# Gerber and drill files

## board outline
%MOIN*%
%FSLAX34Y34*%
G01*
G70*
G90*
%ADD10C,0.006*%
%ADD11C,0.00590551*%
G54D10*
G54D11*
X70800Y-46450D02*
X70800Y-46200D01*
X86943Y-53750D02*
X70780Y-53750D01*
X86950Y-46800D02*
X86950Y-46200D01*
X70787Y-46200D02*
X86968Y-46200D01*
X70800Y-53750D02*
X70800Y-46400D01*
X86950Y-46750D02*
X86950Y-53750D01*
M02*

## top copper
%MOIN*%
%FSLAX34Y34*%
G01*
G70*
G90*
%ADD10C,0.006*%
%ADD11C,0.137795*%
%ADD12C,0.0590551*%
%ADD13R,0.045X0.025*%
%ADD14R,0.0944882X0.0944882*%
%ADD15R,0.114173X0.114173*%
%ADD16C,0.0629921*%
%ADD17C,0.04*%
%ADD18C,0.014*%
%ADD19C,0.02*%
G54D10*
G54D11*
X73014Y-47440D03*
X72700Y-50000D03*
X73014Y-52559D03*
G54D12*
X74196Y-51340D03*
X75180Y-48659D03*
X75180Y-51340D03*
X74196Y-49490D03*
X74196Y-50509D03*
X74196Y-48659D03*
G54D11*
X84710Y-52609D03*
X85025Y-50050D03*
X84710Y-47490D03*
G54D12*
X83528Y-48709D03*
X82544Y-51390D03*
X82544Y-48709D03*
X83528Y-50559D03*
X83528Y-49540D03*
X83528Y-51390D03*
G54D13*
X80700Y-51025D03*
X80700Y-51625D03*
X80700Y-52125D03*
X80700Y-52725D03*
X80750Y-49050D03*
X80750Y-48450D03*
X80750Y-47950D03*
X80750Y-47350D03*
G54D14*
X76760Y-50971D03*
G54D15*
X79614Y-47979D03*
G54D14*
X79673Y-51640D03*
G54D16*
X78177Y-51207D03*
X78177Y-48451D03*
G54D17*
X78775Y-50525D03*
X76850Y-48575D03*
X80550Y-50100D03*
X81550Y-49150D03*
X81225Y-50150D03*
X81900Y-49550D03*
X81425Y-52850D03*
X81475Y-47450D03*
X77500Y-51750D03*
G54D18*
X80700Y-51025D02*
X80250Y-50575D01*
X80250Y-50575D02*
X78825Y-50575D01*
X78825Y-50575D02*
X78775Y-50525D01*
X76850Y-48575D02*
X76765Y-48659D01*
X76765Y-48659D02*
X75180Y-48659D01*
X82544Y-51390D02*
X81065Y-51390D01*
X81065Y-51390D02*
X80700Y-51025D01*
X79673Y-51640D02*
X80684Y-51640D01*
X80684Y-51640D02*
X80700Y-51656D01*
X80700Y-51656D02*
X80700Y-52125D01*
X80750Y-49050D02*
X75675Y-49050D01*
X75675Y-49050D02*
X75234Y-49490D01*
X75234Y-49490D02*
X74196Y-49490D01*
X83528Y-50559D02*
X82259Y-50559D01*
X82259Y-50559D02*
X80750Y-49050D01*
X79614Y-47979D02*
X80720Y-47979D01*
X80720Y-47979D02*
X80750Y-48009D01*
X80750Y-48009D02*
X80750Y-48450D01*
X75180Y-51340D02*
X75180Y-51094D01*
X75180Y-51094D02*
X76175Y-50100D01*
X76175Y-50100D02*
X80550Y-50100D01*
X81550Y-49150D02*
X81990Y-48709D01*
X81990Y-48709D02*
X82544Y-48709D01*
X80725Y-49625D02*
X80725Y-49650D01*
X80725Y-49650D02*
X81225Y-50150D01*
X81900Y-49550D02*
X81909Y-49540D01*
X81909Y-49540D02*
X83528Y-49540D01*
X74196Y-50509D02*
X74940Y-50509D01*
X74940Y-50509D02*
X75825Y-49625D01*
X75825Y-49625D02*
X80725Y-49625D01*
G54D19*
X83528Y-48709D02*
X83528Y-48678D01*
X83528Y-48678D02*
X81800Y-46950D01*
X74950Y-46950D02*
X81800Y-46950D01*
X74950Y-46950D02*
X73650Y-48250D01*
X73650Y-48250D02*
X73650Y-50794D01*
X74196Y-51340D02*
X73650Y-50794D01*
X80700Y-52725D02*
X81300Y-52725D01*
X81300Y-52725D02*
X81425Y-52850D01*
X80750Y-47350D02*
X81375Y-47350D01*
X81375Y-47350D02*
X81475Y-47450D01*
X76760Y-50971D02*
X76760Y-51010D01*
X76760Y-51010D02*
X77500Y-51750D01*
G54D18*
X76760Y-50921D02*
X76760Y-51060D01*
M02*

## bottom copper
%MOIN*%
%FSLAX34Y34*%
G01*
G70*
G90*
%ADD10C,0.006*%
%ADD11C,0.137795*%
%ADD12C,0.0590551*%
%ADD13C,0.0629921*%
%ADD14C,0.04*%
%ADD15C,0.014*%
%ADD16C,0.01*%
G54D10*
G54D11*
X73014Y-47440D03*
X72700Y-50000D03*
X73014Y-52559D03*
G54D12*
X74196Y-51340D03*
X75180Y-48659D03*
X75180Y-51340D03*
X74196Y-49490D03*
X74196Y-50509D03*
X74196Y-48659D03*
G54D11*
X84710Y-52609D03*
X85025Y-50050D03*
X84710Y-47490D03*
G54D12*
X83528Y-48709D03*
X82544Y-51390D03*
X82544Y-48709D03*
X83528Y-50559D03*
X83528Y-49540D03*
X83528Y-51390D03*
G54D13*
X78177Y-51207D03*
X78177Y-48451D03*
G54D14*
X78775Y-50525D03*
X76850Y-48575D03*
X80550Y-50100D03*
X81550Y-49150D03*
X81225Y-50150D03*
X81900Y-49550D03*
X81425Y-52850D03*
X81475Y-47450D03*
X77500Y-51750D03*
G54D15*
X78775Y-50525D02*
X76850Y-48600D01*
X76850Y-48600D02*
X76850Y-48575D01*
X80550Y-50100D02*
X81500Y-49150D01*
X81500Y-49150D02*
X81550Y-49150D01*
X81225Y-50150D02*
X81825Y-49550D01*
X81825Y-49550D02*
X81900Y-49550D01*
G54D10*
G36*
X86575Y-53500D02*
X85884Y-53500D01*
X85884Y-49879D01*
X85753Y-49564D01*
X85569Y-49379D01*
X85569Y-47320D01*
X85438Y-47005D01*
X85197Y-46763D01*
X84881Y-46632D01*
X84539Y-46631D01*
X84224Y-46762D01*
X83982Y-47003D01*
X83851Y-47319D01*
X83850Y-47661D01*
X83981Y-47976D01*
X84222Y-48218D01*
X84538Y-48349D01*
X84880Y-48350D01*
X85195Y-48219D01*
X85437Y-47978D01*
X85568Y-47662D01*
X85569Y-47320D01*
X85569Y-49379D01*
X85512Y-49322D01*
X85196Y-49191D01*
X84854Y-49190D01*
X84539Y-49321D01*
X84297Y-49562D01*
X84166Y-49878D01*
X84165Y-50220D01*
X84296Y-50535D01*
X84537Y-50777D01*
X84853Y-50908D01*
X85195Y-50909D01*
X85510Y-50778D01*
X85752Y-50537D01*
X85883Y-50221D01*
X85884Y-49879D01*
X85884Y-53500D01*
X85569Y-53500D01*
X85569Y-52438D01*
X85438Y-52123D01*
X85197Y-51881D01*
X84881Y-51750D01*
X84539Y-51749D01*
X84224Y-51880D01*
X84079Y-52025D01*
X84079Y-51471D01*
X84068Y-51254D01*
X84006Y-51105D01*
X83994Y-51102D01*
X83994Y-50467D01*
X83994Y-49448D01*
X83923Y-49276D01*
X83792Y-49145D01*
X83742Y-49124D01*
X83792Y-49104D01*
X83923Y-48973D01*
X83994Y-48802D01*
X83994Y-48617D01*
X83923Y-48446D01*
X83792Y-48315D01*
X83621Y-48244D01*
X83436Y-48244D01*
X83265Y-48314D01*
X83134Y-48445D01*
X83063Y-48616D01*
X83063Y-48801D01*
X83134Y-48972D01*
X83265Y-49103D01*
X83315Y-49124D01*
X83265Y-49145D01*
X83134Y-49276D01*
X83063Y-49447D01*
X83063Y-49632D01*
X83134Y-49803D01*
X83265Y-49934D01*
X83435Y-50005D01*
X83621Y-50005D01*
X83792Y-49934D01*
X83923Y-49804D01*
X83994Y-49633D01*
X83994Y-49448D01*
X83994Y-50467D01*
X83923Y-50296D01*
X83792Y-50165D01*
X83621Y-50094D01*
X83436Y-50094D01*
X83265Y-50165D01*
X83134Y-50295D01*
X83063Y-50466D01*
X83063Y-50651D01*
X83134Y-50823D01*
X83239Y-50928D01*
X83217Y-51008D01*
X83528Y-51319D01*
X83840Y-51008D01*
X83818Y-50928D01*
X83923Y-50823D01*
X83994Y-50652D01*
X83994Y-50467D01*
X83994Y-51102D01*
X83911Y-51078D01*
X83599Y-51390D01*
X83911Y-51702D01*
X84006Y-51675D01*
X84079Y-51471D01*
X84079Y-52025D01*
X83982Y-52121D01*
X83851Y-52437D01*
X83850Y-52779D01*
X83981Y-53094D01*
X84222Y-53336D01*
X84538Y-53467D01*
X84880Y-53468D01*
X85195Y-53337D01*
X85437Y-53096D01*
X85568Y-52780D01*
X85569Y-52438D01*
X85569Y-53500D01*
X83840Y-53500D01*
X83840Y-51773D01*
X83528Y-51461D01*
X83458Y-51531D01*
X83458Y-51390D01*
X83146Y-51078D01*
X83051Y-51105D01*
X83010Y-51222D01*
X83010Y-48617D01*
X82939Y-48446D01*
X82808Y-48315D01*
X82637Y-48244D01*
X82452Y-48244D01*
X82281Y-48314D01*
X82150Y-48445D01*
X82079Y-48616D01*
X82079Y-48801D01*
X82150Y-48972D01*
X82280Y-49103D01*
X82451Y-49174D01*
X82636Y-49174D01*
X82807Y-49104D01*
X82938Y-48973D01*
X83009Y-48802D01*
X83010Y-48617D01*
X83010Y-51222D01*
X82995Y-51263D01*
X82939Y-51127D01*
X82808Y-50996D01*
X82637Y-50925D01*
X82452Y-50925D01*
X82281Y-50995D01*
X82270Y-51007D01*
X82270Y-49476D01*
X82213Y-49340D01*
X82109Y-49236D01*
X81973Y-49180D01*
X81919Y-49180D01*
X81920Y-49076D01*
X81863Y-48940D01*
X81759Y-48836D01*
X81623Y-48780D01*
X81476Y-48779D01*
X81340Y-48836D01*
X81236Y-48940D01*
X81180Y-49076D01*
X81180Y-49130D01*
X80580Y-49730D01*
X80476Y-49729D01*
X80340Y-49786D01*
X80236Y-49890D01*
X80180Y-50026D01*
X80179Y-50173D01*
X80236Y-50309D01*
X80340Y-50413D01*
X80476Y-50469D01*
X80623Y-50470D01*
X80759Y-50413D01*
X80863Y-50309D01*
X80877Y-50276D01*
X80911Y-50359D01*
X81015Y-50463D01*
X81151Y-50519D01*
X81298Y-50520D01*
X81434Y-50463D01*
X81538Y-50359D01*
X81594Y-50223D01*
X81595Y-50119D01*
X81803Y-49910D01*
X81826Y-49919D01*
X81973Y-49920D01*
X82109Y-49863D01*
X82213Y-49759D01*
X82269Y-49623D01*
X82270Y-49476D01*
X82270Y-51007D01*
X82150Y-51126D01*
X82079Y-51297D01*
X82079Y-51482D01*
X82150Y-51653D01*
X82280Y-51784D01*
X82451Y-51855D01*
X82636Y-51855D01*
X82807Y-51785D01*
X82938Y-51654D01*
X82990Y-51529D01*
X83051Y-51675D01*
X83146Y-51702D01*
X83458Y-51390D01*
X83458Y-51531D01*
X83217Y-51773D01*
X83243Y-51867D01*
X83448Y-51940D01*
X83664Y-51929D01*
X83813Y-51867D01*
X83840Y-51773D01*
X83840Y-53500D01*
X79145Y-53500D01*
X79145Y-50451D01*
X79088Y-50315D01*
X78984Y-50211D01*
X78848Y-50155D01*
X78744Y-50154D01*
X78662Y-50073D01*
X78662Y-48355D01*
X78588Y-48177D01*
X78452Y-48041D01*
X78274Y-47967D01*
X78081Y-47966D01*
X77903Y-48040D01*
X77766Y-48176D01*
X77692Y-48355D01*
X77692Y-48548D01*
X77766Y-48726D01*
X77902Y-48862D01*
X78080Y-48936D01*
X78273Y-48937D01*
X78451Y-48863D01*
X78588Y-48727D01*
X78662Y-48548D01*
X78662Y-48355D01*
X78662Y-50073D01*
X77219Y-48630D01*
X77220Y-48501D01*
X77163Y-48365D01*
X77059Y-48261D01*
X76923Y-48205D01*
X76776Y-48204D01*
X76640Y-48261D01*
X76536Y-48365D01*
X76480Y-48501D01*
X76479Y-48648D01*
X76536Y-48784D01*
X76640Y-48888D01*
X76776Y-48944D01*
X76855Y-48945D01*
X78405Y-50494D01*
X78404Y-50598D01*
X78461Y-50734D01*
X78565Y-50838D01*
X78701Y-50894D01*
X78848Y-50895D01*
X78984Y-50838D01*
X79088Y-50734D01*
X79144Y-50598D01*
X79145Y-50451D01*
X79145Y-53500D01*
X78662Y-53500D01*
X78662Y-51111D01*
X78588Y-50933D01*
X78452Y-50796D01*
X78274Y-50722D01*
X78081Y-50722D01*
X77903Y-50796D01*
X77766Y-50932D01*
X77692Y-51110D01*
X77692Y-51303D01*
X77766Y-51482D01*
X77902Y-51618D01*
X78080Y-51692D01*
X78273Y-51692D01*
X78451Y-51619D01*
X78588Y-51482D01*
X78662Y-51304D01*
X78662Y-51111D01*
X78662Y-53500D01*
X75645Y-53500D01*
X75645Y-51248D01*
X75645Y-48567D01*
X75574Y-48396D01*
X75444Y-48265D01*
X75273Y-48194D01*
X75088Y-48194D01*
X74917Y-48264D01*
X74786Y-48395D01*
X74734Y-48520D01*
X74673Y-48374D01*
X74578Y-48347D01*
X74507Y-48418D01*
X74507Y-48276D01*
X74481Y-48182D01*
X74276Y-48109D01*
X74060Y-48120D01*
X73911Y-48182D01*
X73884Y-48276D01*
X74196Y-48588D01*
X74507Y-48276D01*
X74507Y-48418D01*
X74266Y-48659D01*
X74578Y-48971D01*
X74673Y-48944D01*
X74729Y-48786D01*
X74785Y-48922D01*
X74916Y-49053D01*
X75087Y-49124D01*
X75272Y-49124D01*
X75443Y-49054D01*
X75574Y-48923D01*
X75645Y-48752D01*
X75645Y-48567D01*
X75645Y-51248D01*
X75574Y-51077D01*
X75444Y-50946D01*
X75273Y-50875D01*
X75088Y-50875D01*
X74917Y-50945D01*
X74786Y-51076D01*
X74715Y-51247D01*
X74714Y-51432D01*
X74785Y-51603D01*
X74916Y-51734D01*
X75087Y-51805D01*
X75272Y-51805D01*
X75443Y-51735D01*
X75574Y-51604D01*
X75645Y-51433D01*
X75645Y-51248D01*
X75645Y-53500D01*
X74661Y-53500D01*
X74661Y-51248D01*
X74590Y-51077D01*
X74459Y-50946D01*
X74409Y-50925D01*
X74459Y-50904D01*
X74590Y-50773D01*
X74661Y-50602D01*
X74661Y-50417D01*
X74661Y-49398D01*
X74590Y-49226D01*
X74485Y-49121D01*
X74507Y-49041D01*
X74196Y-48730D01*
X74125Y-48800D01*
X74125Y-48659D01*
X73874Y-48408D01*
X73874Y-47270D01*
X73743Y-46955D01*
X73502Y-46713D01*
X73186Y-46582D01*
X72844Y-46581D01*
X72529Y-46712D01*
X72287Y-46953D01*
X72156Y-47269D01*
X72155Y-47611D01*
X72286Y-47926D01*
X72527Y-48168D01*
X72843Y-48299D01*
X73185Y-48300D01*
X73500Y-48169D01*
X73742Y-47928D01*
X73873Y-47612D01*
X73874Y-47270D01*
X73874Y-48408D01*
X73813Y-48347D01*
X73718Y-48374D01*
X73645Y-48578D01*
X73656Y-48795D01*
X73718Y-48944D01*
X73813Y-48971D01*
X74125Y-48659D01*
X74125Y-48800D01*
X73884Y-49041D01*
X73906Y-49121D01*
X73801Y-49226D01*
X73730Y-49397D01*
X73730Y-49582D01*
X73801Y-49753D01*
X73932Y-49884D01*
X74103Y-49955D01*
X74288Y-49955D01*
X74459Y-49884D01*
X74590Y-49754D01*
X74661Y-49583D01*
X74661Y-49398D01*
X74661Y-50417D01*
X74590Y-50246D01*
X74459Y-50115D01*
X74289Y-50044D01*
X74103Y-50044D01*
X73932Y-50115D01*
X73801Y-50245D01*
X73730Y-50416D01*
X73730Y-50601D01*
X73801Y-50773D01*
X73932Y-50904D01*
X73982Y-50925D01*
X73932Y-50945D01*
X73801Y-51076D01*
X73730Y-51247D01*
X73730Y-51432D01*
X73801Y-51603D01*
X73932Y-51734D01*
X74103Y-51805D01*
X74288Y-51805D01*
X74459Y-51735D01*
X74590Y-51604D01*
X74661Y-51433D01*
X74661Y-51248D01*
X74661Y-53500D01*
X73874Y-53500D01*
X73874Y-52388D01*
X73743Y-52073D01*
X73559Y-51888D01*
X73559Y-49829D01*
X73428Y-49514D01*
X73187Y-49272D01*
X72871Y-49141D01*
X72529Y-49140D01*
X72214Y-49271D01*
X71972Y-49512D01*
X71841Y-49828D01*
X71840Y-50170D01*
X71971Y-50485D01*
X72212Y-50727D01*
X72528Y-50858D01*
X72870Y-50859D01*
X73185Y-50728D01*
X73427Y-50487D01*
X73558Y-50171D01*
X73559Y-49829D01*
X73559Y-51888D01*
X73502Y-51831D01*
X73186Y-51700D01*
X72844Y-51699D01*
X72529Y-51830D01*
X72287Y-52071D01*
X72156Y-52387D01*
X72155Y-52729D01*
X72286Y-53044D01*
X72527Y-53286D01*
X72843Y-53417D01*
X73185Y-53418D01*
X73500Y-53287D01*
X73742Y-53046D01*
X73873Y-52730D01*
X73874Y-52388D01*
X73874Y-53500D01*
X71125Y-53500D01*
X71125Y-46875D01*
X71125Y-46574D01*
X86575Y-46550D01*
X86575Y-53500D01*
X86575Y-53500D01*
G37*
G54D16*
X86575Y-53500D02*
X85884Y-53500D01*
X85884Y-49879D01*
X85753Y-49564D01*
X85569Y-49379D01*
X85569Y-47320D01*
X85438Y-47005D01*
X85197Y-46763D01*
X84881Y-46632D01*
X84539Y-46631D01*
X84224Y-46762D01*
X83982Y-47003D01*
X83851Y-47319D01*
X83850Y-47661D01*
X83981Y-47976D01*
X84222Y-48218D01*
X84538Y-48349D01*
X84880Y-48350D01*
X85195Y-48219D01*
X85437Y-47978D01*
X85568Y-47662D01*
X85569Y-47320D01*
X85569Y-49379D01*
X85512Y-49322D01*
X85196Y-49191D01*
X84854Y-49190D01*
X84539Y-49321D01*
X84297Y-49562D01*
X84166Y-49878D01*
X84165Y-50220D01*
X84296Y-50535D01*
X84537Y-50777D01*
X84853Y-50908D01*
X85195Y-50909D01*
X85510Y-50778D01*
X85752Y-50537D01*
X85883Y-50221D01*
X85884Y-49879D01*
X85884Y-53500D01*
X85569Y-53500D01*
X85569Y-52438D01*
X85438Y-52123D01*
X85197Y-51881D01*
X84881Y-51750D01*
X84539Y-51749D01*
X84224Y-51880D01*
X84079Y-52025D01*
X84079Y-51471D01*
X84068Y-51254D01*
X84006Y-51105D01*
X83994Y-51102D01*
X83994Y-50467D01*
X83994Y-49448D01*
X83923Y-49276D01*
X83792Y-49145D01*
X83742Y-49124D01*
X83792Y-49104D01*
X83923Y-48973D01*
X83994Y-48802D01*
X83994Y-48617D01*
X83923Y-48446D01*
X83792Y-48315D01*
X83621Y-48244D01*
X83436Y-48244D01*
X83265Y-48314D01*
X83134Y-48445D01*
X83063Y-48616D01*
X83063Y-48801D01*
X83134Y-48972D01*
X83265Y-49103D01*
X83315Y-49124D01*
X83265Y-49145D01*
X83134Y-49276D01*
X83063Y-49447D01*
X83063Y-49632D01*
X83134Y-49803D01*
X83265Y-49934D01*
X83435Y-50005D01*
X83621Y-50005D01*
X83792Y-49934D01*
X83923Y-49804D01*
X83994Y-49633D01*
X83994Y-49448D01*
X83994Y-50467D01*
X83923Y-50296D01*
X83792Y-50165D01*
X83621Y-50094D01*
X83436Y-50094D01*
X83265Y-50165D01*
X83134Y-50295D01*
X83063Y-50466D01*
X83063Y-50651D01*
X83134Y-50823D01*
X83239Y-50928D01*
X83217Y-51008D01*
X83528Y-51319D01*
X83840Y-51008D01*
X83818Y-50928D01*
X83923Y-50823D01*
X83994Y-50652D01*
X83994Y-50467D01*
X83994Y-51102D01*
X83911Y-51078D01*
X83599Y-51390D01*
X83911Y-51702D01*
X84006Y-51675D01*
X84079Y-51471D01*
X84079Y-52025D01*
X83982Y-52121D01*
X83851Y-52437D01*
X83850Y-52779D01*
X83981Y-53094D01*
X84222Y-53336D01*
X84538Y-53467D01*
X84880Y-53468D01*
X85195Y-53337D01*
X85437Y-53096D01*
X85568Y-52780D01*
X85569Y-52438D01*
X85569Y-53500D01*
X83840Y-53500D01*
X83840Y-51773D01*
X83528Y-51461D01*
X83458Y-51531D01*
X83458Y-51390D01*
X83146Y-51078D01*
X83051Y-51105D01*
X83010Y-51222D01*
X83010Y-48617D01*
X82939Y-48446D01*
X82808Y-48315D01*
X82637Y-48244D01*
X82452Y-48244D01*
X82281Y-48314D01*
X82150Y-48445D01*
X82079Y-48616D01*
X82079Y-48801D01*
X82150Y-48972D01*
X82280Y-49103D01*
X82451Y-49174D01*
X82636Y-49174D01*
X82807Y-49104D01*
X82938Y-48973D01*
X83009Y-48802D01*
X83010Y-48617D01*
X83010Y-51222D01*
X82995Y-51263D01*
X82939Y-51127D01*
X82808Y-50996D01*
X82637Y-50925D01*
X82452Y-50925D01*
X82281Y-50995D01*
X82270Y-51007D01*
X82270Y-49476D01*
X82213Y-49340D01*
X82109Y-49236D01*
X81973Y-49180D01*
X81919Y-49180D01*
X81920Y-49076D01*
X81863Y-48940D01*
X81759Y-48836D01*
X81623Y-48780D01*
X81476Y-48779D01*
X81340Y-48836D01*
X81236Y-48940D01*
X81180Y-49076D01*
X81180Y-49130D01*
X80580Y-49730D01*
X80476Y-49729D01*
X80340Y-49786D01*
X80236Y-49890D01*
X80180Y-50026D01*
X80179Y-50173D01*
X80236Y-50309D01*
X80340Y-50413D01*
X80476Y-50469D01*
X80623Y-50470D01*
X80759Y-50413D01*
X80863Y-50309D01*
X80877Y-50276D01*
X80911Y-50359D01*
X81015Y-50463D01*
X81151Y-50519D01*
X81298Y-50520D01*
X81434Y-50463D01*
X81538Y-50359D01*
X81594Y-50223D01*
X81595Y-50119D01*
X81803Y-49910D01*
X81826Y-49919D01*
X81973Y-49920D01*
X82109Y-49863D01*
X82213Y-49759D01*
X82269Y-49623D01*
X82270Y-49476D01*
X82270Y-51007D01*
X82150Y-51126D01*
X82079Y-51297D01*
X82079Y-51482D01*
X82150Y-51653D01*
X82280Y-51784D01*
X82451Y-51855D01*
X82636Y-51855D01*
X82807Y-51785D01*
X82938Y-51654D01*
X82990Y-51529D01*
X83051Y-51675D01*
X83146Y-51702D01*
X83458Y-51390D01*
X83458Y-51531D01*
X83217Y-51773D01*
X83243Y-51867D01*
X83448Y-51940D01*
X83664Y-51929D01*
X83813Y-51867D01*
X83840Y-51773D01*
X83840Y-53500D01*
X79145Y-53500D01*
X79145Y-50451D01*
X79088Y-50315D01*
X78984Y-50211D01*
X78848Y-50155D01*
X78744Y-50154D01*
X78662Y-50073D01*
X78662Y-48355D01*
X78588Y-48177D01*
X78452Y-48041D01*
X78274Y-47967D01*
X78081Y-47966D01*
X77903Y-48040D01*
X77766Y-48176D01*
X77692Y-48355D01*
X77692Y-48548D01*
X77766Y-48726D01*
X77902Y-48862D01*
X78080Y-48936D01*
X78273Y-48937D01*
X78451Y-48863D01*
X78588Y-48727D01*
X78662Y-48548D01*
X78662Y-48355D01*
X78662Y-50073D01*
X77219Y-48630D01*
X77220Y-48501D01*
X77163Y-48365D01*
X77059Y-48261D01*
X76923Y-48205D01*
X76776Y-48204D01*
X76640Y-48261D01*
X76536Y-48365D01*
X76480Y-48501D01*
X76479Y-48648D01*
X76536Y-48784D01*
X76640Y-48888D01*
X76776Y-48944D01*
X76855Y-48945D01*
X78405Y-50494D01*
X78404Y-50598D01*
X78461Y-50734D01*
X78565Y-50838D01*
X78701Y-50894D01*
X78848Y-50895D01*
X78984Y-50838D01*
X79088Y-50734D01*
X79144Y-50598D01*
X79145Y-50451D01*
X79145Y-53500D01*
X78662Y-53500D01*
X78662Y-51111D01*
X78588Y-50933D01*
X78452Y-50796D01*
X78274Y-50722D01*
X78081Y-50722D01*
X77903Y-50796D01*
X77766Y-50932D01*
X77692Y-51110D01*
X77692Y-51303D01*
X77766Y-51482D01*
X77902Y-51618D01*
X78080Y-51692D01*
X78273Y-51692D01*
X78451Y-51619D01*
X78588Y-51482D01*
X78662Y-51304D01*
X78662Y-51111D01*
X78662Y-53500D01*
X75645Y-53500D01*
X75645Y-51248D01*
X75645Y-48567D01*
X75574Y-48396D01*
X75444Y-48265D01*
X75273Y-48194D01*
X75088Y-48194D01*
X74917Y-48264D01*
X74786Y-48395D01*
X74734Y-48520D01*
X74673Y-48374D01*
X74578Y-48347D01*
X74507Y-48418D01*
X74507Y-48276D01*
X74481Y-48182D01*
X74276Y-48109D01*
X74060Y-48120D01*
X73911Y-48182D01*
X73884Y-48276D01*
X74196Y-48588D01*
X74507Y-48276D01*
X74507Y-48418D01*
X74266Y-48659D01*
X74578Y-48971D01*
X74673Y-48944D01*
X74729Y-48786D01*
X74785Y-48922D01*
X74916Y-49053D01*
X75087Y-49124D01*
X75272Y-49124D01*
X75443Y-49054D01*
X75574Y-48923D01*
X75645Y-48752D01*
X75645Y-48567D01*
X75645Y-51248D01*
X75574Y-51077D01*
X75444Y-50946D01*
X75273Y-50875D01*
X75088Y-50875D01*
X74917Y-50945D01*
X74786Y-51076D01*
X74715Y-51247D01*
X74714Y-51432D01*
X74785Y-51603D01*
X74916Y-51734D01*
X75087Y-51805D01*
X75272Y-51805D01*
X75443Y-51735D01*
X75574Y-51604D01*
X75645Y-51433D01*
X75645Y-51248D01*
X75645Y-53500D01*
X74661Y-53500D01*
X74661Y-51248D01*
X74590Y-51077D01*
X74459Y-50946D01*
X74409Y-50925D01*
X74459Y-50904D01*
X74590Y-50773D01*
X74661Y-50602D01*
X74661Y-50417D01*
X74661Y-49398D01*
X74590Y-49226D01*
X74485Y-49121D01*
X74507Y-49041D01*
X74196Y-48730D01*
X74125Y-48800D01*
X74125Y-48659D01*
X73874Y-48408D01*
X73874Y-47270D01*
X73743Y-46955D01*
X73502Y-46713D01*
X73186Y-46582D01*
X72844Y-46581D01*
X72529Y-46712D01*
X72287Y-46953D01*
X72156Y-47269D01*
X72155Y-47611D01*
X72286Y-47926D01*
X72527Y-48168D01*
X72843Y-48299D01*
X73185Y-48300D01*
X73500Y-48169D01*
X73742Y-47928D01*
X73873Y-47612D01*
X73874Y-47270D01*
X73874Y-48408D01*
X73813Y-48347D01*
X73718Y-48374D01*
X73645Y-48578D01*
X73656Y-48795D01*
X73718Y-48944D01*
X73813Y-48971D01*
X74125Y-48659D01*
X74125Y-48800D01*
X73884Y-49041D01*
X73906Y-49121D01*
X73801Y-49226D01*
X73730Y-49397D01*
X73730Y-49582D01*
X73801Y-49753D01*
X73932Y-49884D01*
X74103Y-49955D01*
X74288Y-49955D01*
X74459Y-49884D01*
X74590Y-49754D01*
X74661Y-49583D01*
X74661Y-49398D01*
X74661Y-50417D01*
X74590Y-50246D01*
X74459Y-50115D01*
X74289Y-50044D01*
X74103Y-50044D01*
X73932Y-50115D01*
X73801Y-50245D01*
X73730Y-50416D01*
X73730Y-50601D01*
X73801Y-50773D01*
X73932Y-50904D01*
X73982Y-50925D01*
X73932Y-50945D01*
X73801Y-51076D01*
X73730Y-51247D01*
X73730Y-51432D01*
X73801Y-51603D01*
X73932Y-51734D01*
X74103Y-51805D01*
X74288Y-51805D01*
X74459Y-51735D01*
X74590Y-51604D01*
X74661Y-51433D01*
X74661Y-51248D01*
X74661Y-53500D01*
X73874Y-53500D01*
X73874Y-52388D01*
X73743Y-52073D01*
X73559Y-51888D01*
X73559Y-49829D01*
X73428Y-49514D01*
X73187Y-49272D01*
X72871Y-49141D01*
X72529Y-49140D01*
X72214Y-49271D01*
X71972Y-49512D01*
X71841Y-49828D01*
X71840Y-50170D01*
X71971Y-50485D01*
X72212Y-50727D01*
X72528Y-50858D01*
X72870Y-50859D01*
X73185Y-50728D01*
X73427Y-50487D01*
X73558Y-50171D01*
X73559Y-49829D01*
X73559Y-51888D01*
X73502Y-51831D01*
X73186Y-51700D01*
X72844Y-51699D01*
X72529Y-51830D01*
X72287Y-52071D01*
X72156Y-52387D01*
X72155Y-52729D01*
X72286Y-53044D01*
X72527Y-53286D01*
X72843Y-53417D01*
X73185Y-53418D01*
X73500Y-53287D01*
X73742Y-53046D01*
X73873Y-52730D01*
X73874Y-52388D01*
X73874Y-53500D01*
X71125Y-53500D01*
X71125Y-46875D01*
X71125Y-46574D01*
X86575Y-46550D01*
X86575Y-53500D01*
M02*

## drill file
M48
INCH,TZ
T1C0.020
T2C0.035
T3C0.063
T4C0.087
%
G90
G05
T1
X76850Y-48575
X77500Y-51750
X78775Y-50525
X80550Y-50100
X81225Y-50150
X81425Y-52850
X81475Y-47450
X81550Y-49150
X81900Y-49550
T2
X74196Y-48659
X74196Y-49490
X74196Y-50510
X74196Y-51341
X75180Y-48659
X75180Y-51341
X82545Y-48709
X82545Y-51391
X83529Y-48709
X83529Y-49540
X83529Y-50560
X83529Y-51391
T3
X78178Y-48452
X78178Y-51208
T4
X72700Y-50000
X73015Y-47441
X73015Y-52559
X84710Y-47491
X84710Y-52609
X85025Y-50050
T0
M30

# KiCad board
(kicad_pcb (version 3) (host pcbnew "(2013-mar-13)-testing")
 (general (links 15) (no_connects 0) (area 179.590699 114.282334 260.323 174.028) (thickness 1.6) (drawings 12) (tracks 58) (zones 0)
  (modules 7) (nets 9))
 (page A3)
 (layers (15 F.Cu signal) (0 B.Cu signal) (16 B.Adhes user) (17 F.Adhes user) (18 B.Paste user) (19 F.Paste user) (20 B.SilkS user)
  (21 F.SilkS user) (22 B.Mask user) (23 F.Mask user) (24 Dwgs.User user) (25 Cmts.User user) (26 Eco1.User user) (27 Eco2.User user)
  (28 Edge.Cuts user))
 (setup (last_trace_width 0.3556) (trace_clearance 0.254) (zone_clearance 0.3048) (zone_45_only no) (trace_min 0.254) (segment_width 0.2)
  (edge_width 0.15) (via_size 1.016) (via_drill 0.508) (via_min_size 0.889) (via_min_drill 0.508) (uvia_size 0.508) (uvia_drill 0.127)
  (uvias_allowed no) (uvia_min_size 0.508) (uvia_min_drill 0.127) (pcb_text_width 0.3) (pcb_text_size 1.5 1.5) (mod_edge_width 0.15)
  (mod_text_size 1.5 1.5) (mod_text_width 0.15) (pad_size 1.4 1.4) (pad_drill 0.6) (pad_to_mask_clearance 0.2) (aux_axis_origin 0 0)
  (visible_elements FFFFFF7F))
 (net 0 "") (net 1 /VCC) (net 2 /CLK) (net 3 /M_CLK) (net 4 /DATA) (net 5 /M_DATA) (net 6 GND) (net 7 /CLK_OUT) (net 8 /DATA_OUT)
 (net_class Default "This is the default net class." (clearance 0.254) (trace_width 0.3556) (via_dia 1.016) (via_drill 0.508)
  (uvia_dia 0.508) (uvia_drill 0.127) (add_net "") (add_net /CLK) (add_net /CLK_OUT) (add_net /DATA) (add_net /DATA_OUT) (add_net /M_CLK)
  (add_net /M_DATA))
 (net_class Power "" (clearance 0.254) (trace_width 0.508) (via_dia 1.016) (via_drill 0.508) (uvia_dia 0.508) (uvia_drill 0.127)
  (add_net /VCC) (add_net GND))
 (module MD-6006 (layer F.Cu) (at 184.658 127 90)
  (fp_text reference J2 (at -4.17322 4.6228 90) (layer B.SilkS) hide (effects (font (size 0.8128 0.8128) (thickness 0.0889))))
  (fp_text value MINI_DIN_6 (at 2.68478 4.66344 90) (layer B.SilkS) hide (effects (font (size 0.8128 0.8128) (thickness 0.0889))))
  (pad "" thru_hole circle (at 6.5 0.8 90) (size 3.5 3.5) (drill 2.2) (layers *.Cu F.SilkS F.Mask))
  (pad "" thru_hole circle (at 0 0 90) (size 3.5 3.5) (drill 2.2) (layers *.Cu F.SilkS F.Mask))
  (pad "" thru_hole circle (at -6.5 0.8 90) (size 3.5 3.5) (drill 2.2) (layers *.Cu F.SilkS F.Mask))
  (pad 4 thru_hole circle (at -3.405 3.8 90) (size 1.5 1.5) (drill 0.9) (layers *.Cu *.Mask F.SilkS) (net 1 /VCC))
  (pad 5 thru_hole circle (at 3.405 6.3 90) (size 1.5 1.5) (drill 0.9) (layers *.Cu *.Mask F.SilkS) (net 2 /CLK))
  (pad 6 thru_hole circle (at -3.405 6.3 90) (size 1.5 1.5) (drill 0.9) (layers *.Cu *.Mask F.SilkS) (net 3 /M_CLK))
  (pad 1 thru_hole circle (at 1.295 3.8 90) (size 1.5 1.5) (drill 0.9) (layers *.Cu *.Mask F.SilkS) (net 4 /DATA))
  (pad 2 thru_hole circle (at -1.295 3.8 90) (size 1.5 1.5) (drill 0.9) (layers *.Cu *.Mask F.SilkS) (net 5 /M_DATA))
  (pad 3 thru_hole circle (at 3.405 3.8 90) (size 1.5 1.5) (drill 0.9) (layers *.Cu *.Mask F.SilkS) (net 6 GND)))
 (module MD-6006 (layer F.Cu) (at 215.9635 127.127 270)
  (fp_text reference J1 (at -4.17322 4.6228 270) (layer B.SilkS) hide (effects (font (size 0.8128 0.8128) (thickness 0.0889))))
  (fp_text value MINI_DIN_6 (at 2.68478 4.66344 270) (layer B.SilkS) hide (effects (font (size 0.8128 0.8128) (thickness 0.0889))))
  (pad "" thru_hole circle (at 6.5 0.8 270) (size 3.5 3.5) (drill 2.2) (layers *.Cu F.SilkS F.Mask))
  (pad "" thru_hole circle (at 0 0 270) (size 3.5 3.5) (drill 2.2) (layers *.Cu F.SilkS F.Mask))
  (pad "" thru_hole circle (at -6.5 0.8 270) (size 3.5 3.5) (drill 2.2) (layers *.Cu F.SilkS F.Mask))
  (pad 4 thru_hole circle (at -3.405 3.8 270) (size 1.5 1.5) (drill 0.9) (layers *.Cu *.Mask F.SilkS) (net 1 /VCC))
  (pad 5 thru_hole circle (at 3.405 6.3 270) (size 1.5 1.5) (drill 0.9) (layers *.Cu *.Mask F.SilkS) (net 2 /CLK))
  (pad 6 thru_hole circle (at -3.405 6.3 270) (size 1.5 1.5) (drill 0.9) (layers *.Cu *.Mask F.SilkS) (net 3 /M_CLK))
  (pad 1 thru_hole circle (at 1.295 3.8 270) (size 1.5 1.5) (drill 0.9) (layers *.Cu *.Mask F.SilkS) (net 4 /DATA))
  (pad 2 thru_hole circle (at -1.295 3.8 270) (size 1.5 1.5) (drill 0.9) (layers *.Cu *.Mask F.SilkS) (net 5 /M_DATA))
  (pad 3 thru_hole circle (at 3.405 3.8 270) (size 1.5 1.5) (drill 0.9) (layers *.Cu *.Mask F.SilkS) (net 6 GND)))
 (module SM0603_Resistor (layer F.Cu) (at 204.978 130.3655 270)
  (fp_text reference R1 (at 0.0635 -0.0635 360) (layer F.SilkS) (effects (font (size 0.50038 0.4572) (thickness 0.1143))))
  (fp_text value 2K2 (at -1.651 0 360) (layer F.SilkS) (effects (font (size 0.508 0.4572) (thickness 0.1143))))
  (pad 1 smd rect (at -0.762 0 270) (size 0.635 1.143) (layers F.Cu F.Paste F.Mask) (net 2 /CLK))
  (pad 2 smd rect (at 0.762 0 270) (size 0.635 1.143) (layers F.Cu F.Paste F.Mask) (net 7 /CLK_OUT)))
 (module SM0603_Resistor (layer F.Cu) (at 204.978 133.1595 270)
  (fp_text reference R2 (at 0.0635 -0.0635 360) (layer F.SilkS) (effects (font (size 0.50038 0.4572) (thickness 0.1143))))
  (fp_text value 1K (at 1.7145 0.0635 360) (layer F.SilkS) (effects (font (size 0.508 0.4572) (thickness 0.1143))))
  (pad 1 smd rect (at -0.762 0 270) (size 0.635 1.143) (layers F.Cu F.Paste F.Mask) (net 7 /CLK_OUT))
  (pad 2 smd rect (at 0.762 0 270) (size 0.635 1.143) (layers F.Cu F.Paste F.Mask) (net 6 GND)))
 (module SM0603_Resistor (layer F.Cu) (at 205.105 123.825 90)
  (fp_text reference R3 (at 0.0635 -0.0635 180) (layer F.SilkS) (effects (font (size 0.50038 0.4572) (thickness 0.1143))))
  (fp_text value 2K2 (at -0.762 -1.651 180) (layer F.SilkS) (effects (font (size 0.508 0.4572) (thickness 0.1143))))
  (pad 1 smd rect (at -0.762 0 90) (size 0.635 1.143) (layers F.Cu F.Paste F.Mask) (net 4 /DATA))
  (pad 2 smd rect (at 0.762 0 90) (size 0.635 1.143) (layers F.Cu F.Paste F.Mask) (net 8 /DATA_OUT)))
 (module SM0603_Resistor (layer F.Cu) (at 205.105 121.031 90)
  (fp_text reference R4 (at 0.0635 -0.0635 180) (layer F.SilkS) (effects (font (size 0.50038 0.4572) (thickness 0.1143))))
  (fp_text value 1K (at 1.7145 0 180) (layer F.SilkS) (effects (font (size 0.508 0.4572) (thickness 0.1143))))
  (pad 1 smd rect (at -0.762 0 90) (size 0.635 1.143) (layers F.Cu F.Paste F.Mask) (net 8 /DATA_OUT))
  (pad 2 smd rect (at 0.762 0 90) (size 0.635 1.143) (layers F.Cu F.Paste F.Mask) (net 6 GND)))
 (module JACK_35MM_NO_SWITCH (layer F.Cu) (at 198.501 126.238 90)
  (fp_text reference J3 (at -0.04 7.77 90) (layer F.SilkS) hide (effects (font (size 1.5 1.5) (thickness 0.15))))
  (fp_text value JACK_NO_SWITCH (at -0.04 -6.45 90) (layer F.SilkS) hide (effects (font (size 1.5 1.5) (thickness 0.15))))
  (pad 1 smd rect (at -3.23 -3.53 90) (size 2.4 2.4) (layers F.Cu F.Paste F.Mask) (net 6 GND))
  (pad 2 smd rect (at 4.37 3.72 90) (size 2.9 2.9) (layers F.Cu F.Paste F.Mask) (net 8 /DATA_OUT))
  (pad 3 smd rect (at -4.93 3.87 90) (size 2.4 2.4) (layers F.Cu F.Paste F.Mask) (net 7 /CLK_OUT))
  (pad "" thru_hole circle (at -3.83 0.07 90) (size 1.6 1.6) (drill 1.6) (layers *.Cu *.Mask F.SilkS))
  (pad "" thru_hole circle (at 3.17 0.07 90) (size 1.6 1.6) (drill 1.6) (layers *.Cu *.Mask F.SilkS)))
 (gr_line (start 179.832 117.983) (end 179.832 117.348) (angle 90) (layer Edge.Cuts) (width 0.15))
 (gr_line (start 220.8365 136.525) (end 179.7812 136.525) (angle 90) (layer Edge.Cuts) (width 0.15))
 (gr_line (start 220.853 118.872) (end 220.853 117.348) (angle 90) (layer Edge.Cuts) (width 0.15))
 (gr_line (start 179.8 117.348) (end 220.9 117.348) (angle 90) (layer Edge.Cuts) (width 0.15))
 (gr_line (start 179.832 136.525) (end 179.832 117.856) (angle 90) (layer Edge.Cuts) (width 0.15))
 (gr_line (start 220.853 118.745) (end 220.853 136.525) (angle 90) (layer Edge.Cuts) (width 0.15))
 (segment (start 204.978 129.6035) (end 203.835 128.4605) (width 0.3556) (layer F.Cu) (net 2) (status 10))
 (segment (start 203.835 128.4605) (end 200.2155 128.4605) (width 0.3556) (layer F.Cu) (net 2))
 (segment (start 200.2155 128.4605) (end 200.0885 128.3335) (width 0.3556) (layer F.Cu) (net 2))
 (via (at 200.0885 128.3335) (size 1.016) (layers F.Cu B.Cu) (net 2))
 (segment (start 200.0885 128.3335) (end 195.199 123.444) (width 0.3556) (layer B.Cu) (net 2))
 (segment (start 195.199 123.444) (end 195.199 123.3805) (width 0.3556) (layer B.Cu) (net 2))
 (via (at 195.199 123.3805) (size 1.016) (layers F.Cu B.Cu) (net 2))
 (segment (start 195.199 123.3805) (end 194.9845 123.595) (width 0.3556) (layer F.Cu) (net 2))
 (segment (start 194.9845 123.595) (end 190.958 123.595) (width 0.3556) (layer F.Cu) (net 2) (status 20))
 (segment (start 209.6635 130.532) (end 205.9065 130.532) (width 0.3556) (layer F.Cu) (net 2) (status 10))
 (segment (start 205.9065 130.532) (end 204.978 129.6035) (width 0.3556) (layer F.Cu) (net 2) (status 20))
 (segment (start 202.371 131.168) (end 204.9375 131.168) (width 0.3556) (layer F.Cu) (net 7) (status 30))
 (segment (start 204.9375 131.168) (end 204.978 131.2085) (width 0.3556) (layer F.Cu) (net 7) (status 30))
 (segment (start 204.978 131.2085) (end 204.978 132.3975) (width 0.3556) (layer F.Cu) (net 7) (status 30))
 (segment (start 205.105 124.587) (end 192.2145 124.587) (width 0.3556) (layer F.Cu) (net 4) (status 10))
 (segment (start 192.2145 124.587) (end 191.0965 125.705) (width 0.3556) (layer F.Cu) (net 4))
 (segment (start 191.0965 125.705) (end 188.458 125.705) (width 0.3556) (layer F.Cu) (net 4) (status 20))
 (segment (start 212.1635 128.422) (end 208.94 128.422) (width 0.3556) (layer F.Cu) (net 4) (status 10))
 (segment (start 208.94 128.422) (end 205.105 124.587) (width 0.3556) (layer F.Cu) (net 4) (status 20))
 (segment (start 202.221 121.868) (end 205.03 121.868) (width 0.3556) (layer F.Cu) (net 8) (status 30))
 (segment (start 205.03 121.868) (end 205.105 121.943) (width 0.3556) (layer F.Cu) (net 8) (status 30))
 (segment (start 205.105 121.943) (end 205.105 123.063) (width 0.3556) (layer F.Cu) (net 8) (status 30))
 (segment (start 190.958 130.405) (end 190.958 129.7805) (width 0.3556) (layer F.Cu) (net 3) (status 30))
 (segment (start 190.958 129.7805) (end 193.4845 127.254) (width 0.3556) (layer F.Cu) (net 3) (status 10))
 (segment (start 193.4845 127.254) (end 204.597 127.254) (width 0.3556) (layer F.Cu) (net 3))
 (via (at 204.597 127.254) (size 1.016) (layers F.Cu B.Cu) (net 3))
 (segment (start 204.597 127.254) (end 207.01 124.841) (width 0.3556) (layer B.Cu) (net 3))
 (segment (start 207.01 124.841) (end 207.137 124.841) (width 0.3556) (layer B.Cu) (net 3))
 (via (at 207.137 124.841) (size 1.016) (layers F.Cu B.Cu) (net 3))
 (segment (start 207.137 124.841) (end 208.256 123.722) (width 0.3556) (layer F.Cu) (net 3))
 (segment (start 208.256 123.722) (end 209.6635 123.722) (width 0.3556) (layer F.Cu) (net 3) (status 20))
 (segment (start 205.0415 126.0475) (end 205.0415 126.111) (width 0.3556) (layer F.Cu) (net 5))
 (segment (start 205.0415 126.111) (end 206.3115 127.381) (width 0.3556) (layer F.Cu) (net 5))
 (via (at 206.3115 127.381) (size 1.016) (layers F.Cu B.Cu) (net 5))
 (segment (start 206.3115 127.381) (end 207.8355 125.857) (width 0.3556) (layer B.Cu) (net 5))
 (segment (start 207.8355 125.857) (end 208.026 125.857) (width 0.3556) (layer B.Cu) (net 5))
 (via (at 208.026 125.857) (size 1.016) (layers F.Cu B.Cu) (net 5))
 (segment (start 208.026 125.857) (end 208.051 125.832) (width 0.3556) (layer F.Cu) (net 5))
 (segment (start 208.051 125.832) (end 212.1635 125.832) (width 0.3556) (layer F.Cu) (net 5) (status 20))
 (segment (start 188.458 128.295) (end 190.348 128.295) (width 0.3556) (layer F.Cu) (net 5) (status 10))
 (segment (start 190.348 128.295) (end 192.5955 126.0475) (width 0.3556) (layer F.Cu) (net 5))
 (segment (start 192.5955 126.0475) (end 205.0415 126.0475) (width 0.3556) (layer F.Cu) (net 5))
 (segment (start 212.1635 123.722) (end 212.1635 123.6445) (width 0.508) (layer F.Cu) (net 1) (status 30))
 (segment (start 212.1635 123.6445) (end 207.772 119.253) (width 0.508) (layer F.Cu) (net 1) (status 10))
 (segment (start 190.373 119.253) (end 207.772 119.253) (width 0.508) (layer F.Cu) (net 1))
 (segment (start 190.373 119.253) (end 187.071 122.555) (width 0.508) (layer F.Cu) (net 1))
 (segment (start 187.071 122.555) (end 187.071 129.018) (width 0.508) (layer F.Cu) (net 1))
 (segment (start 188.458 130.405) (end 187.071 129.018) (width 0.508) (layer F.Cu) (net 1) (status 10))
 (segment (start 204.978 133.9215) (end 206.502 133.9215) (width 0.508) (layer F.Cu) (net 6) (status 10))
 (segment (start 206.502 133.9215) (end 206.8195 134.239) (width 0.508) (layer F.Cu) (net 6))
 (via (at 206.8195 134.239) (size 1.016) (layers F.Cu B.Cu) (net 6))
 (segment (start 205.105 120.269) (end 206.6925 120.269) (width 0.508) (layer F.Cu) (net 6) (status 10))
 (segment (start 206.6925 120.269) (end 206.9465 120.523) (width 0.508) (layer F.Cu) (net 6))
 (via (at 206.9465 120.523) (size 1.016) (layers F.Cu B.Cu) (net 6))
 (segment (start 194.971 129.468) (end 194.971 129.566) (width 0.508) (layer F.Cu) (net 6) (status 30))
 (segment (start 194.971 129.566) (end 196.85 131.445) (width 0.508) (layer F.Cu) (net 6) (status 10))
 (via (at 196.85 131.445) (size 1.016) (layers F.Cu B.Cu) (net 6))
 (segment (start 194.971 129.341) (end 194.971 129.693) (width 0.3556) (layer F.Cu) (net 6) (status 30))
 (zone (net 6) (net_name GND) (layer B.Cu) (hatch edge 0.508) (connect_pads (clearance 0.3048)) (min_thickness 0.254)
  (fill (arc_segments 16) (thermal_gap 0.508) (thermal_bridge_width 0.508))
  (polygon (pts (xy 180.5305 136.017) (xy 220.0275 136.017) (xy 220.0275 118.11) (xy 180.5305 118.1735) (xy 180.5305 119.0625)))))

